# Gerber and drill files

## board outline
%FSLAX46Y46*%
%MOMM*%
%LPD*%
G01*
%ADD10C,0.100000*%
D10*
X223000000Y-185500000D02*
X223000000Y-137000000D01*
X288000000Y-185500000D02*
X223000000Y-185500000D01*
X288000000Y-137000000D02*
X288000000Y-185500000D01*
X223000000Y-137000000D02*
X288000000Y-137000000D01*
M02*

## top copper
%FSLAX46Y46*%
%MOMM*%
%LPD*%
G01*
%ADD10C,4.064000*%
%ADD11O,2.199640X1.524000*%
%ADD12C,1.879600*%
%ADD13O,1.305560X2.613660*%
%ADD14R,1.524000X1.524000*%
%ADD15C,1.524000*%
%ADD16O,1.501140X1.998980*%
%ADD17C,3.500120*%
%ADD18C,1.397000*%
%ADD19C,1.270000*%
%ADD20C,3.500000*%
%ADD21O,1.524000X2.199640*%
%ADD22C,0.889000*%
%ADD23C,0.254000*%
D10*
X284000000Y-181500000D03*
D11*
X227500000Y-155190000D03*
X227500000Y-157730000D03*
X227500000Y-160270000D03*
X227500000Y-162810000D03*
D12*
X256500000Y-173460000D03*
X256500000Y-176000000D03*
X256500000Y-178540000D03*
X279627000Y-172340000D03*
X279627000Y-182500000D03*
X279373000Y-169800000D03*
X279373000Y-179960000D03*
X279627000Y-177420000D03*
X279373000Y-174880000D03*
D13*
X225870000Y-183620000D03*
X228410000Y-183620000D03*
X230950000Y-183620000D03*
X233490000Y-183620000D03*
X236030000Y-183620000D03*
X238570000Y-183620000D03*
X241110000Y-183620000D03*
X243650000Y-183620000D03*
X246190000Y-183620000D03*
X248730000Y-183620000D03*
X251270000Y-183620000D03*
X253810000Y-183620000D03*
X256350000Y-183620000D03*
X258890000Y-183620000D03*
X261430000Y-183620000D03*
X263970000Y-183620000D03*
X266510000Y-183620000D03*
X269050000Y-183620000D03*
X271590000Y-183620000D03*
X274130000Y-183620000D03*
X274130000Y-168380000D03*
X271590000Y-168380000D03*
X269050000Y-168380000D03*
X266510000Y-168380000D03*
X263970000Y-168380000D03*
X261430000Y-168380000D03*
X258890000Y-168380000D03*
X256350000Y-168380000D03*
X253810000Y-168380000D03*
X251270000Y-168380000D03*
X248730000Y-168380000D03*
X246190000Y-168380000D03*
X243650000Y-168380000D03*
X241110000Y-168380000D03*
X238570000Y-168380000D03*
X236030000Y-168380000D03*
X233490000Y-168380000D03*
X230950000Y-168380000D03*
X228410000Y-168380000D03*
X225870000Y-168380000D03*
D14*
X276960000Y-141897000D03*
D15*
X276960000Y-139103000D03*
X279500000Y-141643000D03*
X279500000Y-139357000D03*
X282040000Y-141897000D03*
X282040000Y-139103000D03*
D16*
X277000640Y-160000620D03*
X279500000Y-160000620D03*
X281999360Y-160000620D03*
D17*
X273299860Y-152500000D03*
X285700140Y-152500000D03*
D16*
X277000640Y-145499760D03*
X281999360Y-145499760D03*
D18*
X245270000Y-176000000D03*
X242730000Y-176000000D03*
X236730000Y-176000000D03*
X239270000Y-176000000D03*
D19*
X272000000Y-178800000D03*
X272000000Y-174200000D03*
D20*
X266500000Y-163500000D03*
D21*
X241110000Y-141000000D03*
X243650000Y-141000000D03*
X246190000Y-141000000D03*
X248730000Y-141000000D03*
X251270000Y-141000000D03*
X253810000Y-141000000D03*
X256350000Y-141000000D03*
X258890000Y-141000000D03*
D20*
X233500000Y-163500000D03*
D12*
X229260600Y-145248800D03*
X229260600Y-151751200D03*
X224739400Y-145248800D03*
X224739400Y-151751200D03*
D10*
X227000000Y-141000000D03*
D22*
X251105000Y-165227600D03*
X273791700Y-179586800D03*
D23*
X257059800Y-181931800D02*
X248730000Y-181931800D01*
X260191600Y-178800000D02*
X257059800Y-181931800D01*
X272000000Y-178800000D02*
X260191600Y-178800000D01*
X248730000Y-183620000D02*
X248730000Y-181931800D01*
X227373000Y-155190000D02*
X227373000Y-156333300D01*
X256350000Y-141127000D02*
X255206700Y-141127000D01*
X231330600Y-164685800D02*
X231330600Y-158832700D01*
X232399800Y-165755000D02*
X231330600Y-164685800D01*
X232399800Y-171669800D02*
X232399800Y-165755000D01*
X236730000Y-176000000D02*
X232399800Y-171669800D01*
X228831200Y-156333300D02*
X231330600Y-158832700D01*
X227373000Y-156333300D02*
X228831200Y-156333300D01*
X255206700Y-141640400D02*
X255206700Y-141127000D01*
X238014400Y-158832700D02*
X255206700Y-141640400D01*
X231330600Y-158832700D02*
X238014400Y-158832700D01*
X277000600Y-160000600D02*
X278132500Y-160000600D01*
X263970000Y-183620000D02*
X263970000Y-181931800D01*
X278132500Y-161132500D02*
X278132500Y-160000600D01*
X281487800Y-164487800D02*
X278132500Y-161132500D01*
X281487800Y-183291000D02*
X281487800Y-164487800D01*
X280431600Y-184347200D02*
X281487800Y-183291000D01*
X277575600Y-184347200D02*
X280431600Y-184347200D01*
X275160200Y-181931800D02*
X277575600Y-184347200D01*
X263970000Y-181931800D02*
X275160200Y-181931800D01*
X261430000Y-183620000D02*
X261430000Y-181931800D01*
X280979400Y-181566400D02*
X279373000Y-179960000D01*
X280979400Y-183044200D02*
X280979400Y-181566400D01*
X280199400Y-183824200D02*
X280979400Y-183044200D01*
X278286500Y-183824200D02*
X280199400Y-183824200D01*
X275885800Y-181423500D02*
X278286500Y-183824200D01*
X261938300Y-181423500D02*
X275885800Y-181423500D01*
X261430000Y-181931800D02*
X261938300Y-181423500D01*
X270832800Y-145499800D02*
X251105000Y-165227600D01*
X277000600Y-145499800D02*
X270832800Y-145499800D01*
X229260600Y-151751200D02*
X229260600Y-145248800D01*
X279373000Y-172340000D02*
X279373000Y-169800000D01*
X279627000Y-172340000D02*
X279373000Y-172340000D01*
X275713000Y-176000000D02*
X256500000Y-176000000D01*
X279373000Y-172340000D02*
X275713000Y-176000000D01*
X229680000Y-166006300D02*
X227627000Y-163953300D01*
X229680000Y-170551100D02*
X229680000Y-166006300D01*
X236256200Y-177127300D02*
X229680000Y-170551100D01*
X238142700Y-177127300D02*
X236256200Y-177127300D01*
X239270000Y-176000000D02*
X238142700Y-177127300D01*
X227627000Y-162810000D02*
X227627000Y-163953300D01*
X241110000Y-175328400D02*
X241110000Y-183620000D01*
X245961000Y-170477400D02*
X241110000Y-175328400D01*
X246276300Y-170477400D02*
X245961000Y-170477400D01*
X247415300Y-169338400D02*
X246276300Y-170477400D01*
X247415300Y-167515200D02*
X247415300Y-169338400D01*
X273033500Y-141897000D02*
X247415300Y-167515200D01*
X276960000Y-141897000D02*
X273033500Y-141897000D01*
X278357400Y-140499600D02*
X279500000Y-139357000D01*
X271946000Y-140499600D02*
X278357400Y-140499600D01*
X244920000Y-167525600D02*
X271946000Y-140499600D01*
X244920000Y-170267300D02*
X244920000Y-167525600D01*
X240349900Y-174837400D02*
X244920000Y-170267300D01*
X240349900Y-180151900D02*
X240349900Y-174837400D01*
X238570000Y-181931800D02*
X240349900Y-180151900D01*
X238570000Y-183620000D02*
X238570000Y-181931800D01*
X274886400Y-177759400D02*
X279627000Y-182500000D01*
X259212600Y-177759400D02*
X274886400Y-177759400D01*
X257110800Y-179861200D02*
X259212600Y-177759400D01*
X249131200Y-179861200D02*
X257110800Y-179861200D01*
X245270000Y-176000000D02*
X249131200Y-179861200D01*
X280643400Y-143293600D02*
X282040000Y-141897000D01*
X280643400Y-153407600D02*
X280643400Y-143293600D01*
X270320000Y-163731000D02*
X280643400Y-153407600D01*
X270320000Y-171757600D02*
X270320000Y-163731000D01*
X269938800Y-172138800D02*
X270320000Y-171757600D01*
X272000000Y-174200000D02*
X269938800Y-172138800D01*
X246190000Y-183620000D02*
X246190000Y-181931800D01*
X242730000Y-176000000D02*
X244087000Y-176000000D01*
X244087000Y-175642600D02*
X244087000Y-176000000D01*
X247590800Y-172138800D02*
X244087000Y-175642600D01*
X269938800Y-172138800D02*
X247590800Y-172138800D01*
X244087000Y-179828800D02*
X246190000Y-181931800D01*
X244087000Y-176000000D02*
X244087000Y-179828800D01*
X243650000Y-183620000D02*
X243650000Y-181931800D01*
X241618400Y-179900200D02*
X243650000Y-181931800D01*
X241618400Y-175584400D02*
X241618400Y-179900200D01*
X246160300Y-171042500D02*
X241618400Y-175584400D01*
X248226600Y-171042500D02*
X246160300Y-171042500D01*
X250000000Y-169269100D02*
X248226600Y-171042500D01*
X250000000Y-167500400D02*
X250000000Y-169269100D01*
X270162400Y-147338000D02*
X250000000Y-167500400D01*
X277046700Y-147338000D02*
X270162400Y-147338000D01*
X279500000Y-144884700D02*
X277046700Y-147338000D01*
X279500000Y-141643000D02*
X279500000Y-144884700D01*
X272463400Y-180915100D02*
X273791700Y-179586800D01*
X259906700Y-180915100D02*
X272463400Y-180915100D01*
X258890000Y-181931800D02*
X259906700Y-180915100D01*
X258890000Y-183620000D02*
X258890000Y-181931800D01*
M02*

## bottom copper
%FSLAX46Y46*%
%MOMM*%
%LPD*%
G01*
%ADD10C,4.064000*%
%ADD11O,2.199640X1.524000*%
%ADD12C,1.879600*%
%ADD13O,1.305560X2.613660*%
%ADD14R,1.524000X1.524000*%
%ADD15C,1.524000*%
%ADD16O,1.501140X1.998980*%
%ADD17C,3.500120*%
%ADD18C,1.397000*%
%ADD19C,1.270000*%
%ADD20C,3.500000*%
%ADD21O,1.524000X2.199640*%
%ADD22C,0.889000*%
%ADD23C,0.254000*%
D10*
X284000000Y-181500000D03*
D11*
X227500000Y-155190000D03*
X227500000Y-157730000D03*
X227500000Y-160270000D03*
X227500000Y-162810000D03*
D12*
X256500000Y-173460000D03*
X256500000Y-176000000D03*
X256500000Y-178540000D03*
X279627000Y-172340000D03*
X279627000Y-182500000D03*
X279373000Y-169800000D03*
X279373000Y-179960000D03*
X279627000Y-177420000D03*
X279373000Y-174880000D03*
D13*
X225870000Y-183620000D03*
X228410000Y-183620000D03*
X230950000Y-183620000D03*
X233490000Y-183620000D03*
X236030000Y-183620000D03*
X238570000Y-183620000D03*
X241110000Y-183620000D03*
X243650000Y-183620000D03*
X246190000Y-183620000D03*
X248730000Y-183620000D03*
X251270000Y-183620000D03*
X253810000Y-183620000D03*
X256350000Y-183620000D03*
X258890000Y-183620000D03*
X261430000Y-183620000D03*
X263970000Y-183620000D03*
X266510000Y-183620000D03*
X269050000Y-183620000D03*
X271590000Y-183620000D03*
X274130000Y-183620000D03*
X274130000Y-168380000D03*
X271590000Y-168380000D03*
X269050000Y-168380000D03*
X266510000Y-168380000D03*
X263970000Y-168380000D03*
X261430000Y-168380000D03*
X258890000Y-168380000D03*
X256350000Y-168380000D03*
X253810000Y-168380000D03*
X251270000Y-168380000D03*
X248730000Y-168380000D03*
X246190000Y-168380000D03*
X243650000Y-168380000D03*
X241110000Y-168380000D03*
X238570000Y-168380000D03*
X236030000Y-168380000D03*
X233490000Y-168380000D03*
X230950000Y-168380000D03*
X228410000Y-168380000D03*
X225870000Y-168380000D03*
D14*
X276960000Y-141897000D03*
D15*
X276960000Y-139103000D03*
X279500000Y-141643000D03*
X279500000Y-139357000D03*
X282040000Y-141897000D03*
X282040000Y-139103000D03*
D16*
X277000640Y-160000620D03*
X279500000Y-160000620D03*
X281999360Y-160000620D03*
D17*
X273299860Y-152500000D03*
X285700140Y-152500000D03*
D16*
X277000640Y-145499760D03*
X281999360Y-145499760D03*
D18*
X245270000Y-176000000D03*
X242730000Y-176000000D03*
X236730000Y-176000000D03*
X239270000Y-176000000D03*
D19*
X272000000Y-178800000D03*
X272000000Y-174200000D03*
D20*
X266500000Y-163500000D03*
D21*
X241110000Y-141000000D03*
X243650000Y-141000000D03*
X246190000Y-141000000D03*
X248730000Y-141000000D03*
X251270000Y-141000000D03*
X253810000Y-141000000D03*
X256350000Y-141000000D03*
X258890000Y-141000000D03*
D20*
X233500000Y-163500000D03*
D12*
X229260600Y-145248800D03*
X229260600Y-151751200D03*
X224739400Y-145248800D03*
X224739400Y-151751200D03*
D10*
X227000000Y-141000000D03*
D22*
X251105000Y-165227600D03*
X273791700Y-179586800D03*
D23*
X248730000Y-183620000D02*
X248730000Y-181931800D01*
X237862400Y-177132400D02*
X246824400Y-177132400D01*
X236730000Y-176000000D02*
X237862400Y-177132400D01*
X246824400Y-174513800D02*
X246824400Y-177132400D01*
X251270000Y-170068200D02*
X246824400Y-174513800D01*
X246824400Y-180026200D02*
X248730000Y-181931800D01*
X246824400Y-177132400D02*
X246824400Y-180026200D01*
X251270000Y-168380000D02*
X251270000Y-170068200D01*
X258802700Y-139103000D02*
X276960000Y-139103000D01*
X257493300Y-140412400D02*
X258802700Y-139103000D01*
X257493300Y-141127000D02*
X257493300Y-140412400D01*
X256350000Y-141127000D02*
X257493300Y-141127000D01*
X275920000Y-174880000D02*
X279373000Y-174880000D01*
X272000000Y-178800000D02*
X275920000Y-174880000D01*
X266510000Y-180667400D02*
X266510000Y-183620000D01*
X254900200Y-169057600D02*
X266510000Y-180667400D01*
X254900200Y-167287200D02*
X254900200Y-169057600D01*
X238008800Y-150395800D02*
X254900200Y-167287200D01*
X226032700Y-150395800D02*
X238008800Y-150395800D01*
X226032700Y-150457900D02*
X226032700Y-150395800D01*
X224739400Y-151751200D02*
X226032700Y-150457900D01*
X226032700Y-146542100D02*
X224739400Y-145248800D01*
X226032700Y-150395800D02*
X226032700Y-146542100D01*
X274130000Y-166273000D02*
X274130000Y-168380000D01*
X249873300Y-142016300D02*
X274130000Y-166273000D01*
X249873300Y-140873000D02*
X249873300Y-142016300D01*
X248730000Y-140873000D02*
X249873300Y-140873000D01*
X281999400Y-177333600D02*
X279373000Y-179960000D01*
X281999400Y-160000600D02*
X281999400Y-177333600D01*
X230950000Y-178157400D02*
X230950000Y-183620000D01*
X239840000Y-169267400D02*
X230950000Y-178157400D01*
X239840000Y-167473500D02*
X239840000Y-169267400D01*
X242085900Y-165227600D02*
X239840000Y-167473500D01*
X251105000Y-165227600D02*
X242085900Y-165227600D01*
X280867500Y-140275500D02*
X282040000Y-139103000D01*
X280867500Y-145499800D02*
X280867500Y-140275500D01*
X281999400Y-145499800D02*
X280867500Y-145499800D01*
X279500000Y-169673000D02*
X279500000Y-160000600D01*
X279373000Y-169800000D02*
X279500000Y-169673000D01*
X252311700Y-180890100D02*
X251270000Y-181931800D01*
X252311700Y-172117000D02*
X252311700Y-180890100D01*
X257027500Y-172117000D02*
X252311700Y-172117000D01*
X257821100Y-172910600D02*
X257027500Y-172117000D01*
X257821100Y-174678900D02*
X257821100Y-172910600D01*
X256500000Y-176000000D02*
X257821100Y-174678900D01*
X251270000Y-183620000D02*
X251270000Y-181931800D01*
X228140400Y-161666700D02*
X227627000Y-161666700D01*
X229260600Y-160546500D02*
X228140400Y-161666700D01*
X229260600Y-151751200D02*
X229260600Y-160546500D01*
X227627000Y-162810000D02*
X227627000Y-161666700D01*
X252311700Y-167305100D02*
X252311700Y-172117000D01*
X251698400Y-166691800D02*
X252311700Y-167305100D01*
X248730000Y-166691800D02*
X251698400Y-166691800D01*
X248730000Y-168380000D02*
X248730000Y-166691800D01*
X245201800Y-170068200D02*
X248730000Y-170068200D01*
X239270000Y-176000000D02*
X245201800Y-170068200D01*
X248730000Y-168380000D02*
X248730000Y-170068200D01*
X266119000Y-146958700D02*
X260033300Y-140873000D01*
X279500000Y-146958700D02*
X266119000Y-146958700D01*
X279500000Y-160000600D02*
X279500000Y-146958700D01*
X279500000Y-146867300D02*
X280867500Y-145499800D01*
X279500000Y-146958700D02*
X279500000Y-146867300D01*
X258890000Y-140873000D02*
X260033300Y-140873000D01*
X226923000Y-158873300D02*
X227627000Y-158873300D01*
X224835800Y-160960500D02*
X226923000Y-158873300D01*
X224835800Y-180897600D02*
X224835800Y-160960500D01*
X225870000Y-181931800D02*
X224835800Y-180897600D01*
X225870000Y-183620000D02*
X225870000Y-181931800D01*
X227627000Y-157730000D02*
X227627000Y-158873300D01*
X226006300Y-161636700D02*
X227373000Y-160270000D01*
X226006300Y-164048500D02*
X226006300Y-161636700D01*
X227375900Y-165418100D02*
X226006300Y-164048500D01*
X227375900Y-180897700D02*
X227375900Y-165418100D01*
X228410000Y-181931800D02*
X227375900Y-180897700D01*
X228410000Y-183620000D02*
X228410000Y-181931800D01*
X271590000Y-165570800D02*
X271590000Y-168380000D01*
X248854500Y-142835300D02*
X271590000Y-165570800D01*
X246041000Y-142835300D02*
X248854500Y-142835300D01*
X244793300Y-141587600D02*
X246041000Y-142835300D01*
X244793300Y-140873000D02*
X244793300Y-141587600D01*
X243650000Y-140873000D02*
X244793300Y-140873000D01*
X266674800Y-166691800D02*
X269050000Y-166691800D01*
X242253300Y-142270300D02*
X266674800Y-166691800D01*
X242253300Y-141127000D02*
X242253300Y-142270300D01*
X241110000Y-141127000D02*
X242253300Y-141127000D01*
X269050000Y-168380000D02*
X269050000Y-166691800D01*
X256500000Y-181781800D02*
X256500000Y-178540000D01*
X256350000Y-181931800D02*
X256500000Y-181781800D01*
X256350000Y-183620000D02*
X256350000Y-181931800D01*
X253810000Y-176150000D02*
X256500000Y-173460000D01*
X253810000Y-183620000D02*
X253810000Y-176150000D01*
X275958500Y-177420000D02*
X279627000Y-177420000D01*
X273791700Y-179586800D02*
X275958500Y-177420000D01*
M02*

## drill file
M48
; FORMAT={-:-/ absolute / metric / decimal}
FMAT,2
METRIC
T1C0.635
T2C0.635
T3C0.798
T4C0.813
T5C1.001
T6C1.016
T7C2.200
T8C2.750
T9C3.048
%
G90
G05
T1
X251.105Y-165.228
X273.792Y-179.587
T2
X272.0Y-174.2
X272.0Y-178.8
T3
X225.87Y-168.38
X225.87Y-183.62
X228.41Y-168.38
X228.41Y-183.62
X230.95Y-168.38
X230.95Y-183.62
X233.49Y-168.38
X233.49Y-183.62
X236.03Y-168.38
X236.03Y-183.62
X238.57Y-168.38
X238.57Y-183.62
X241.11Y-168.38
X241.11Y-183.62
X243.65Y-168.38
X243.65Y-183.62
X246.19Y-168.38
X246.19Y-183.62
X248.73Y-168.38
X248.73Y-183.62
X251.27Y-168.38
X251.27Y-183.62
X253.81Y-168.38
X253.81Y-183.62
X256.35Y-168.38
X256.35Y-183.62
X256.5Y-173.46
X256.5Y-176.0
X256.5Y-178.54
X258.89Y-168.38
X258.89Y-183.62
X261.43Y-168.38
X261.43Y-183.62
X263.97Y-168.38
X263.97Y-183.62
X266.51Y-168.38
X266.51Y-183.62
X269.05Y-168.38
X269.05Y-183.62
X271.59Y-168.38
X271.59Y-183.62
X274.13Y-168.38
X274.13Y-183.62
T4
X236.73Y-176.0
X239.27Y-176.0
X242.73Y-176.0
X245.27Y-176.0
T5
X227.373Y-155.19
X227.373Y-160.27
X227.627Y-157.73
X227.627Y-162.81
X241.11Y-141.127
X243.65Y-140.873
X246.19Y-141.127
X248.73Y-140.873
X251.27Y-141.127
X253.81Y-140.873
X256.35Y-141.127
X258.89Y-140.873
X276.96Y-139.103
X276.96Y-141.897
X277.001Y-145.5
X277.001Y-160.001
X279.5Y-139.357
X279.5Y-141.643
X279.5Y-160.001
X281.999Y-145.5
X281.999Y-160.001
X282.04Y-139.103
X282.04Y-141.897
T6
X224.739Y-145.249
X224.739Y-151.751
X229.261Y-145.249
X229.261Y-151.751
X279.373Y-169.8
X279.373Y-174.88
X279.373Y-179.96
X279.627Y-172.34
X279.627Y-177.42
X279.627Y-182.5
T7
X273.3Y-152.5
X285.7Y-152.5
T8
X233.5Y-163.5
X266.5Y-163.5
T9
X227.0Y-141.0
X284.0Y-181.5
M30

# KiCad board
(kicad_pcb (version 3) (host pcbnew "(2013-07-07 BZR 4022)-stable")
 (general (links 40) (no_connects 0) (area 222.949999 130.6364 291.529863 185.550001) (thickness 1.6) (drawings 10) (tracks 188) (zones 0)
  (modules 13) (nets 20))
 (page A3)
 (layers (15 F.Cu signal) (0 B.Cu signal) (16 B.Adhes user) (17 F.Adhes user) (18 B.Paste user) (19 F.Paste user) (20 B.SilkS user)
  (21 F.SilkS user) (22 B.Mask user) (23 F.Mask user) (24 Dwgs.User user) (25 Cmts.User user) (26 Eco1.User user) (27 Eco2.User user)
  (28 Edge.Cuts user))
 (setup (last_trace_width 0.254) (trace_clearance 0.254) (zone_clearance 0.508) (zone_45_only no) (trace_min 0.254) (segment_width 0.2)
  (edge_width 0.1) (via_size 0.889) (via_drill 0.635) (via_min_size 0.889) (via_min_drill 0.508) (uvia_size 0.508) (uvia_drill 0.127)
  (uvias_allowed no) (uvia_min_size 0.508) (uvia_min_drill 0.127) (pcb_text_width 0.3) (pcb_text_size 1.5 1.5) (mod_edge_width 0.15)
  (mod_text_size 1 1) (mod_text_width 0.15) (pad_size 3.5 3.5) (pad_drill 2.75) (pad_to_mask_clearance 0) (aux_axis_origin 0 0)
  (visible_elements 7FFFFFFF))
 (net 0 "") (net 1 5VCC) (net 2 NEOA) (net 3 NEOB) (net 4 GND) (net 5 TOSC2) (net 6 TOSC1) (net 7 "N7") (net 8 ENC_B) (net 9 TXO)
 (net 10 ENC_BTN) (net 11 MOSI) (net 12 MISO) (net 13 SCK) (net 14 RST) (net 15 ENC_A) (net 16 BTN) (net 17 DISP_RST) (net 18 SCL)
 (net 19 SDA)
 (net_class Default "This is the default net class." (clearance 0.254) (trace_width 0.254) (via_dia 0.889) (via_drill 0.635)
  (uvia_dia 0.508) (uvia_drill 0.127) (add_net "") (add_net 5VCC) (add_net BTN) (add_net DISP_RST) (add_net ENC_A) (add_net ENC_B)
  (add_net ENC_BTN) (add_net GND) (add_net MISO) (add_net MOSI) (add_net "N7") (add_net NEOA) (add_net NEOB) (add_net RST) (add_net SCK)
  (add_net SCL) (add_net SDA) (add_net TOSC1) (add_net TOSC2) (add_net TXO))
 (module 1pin (layer F.Cu) (at 284 181.5)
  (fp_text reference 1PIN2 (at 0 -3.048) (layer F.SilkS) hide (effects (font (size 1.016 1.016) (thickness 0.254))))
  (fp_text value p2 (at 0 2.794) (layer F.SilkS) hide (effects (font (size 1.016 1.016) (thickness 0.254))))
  (pad 1 thru_hole circle (at 0 0) (size 4.064 4.064) (drill 3.048) (layers *.Cu *.Mask F.SilkS)))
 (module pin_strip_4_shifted (layer F.Cu) (at 227.5 159 270)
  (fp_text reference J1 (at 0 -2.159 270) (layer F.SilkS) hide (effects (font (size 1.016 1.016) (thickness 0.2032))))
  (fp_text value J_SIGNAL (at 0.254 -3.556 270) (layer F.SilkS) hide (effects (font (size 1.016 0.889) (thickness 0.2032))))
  (pad 1 thru_hole oval (at -3.81 0.127 270) (size 1.524 2.19964) (drill 1.00076 (offset 0 -0.127)) (layers *.Cu *.Mask F.SilkS)
   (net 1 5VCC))
  (pad 2 thru_hole oval (at -1.27 -0.127 270) (size 1.524 2.19964) (drill 1.00076 (offset 0 0.127)) (layers *.Cu *.Mask F.SilkS)
   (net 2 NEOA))
  (pad 3 thru_hole oval (at 1.27 0.127 270) (size 1.524 2.19964) (drill 1.00076 (offset 0 -0.127)) (layers *.Cu *.Mask F.SilkS) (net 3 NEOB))
  (pad 4 thru_hole oval (at 3.81 -0.127 270) (size 1.524 2.19964) (drill 1.00076 (offset 0 0.127)) (layers *.Cu *.Mask F.SilkS) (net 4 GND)))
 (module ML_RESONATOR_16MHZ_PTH (layer F.Cu) (at 256.5 176 270)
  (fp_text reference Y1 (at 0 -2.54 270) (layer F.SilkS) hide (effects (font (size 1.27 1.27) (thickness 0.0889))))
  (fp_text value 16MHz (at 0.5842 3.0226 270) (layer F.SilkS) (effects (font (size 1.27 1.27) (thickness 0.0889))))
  (pad 1 thru_hole circle (at -2.54 0 270) (size 1.8796 1.8796) (drill 0.79756) (layers *.Cu *.Mask F.Paste F.SilkS) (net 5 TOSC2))
  (pad 2 thru_hole circle (at 0 0 270) (size 1.8796 1.8796) (drill 0.79756) (layers *.Cu *.Mask F.Paste F.SilkS) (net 4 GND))
  (pad 3 thru_hole circle (at 2.54 0 270) (size 1.8796 1.8796) (drill 0.79756) (layers *.Cu *.Mask F.Paste F.SilkS) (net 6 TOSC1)))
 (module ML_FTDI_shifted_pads (layer F.Cu) (at 279.5 182.5 90)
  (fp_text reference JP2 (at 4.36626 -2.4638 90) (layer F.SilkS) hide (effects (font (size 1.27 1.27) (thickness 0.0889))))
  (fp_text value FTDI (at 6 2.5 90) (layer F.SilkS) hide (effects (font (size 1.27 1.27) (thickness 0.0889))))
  (pad CTS thru_hole circle (at 10.16 0.127 90) (size 1.8796 1.8796) (drill 1.016) (layers *.Cu *.Mask F.Paste F.SilkS) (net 4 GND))
  (pad DTR thru_hole circle (at 0 0.127 90) (size 1.8796 1.8796) (drill 1.016) (layers *.Cu *.Mask F.Paste F.SilkS) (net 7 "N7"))
  (pad GND thru_hole circle (at 12.7 -0.127 90) (size 1.8796 1.8796) (drill 1.016) (layers *.Cu *.Mask F.Paste F.SilkS) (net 4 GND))
  (pad RXI thru_hole circle (at 2.54 -0.127 90) (size 1.8796 1.8796) (drill 1.016) (layers *.Cu *.Mask F.Paste F.SilkS) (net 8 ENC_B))
  (pad TXO thru_hole circle (at 5.08 0.127 90) (size 1.8796 1.8796) (drill 1.016) (layers *.Cu *.Mask F.Paste F.SilkS) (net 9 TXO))
  (pad VCC thru_hole circle (at 7.62 -0.127 90) (size 1.8796 1.8796) (drill 1.016) (layers *.Cu *.Mask F.Paste F.SilkS) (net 1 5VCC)))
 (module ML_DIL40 (layer F.Cu) (at 250 176)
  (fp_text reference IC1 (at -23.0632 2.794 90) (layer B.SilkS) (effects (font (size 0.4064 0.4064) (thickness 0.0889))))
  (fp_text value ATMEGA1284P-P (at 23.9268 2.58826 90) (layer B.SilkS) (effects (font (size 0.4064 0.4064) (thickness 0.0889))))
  (pad 1 thru_hole oval (at -24.13 7.62) (size 1.30556 2.61366) (drill 0.79756) (layers *.Cu *.Mask F.Paste F.SilkS) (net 2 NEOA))
  (pad 2 thru_hole oval (at -21.59 7.62) (size 1.30556 2.61366) (drill 0.79756) (layers *.Cu *.Mask F.Paste F.SilkS) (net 3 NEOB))
  (pad 3 thru_hole oval (at -19.05 7.62) (size 1.30556 2.61366) (drill 0.79756) (layers *.Cu *.Mask F.Paste F.SilkS) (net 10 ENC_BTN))
  (pad 4 thru_hole oval (at -16.51 7.62) (size 1.30556 2.61366) (drill 0.79756) (layers *.Cu *.Mask F.Paste F.SilkS))
  (pad 5 thru_hole oval (at -13.97 7.62) (size 1.30556 2.61366) (drill 0.79756) (layers *.Cu *.Mask F.Paste F.SilkS))
  (pad 6 thru_hole oval (at -11.43 7.62) (size 1.30556 2.61366) (drill 0.79756) (layers *.Cu *.Mask F.Paste F.SilkS) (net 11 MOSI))
  (pad 7 thru_hole oval (at -8.89 7.62) (size 1.30556 2.61366) (drill 0.79756) (layers *.Cu *.Mask F.Paste F.SilkS) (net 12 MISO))
  (pad 8 thru_hole oval (at -6.35 7.62) (size 1.30556 2.61366) (drill 0.79756) (layers *.Cu *.Mask F.Paste F.SilkS) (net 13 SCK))
  (pad 9 thru_hole oval (at -3.81 7.62) (size 1.30556 2.61366) (drill 0.79756) (layers *.Cu *.Mask F.Paste F.SilkS) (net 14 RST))
  (pad 10 thru_hole oval (at -1.27 7.62) (size 1.30556 2.61366) (drill 0.79756) (layers *.Cu *.Mask F.Paste F.SilkS) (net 1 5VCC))
  (pad 11 thru_hole oval (at 1.27 7.62) (size 1.30556 2.61366) (drill 0.79756) (layers *.Cu *.Mask F.Paste F.SilkS) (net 4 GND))
  (pad 12 thru_hole oval (at 3.81 7.62) (size 1.30556 2.61366) (drill 0.79756) (layers *.Cu *.Mask F.Paste F.SilkS) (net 5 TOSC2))
  (pad 13 thru_hole oval (at 6.35 7.62) (size 1.30556 2.61366) (drill 0.79756) (layers *.Cu *.Mask F.Paste F.SilkS) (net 6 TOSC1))
  (pad 14 thru_hole oval (at 8.89 7.62) (size 1.30556 2.61366) (drill 0.79756) (layers *.Cu *.Mask F.Paste F.SilkS) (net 9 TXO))
  (pad 15 thru_hole oval (at 11.43 7.62) (size 1.30556 2.61366) (drill 0.79756) (layers *.Cu *.Mask F.Paste F.SilkS) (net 8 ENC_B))
  (pad 16 thru_hole oval (at 13.97 7.62) (size 1.30556 2.61366) (drill 0.79756) (layers *.Cu *.Mask F.Paste F.SilkS) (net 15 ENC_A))
  (pad 17 thru_hole oval (at 16.51 7.62) (size 1.30556 2.61366) (drill 0.79756) (layers *.Cu *.Mask F.Paste F.SilkS) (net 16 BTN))
  (pad 18 thru_hole oval (at 19.05 7.62) (size 1.30556 2.61366) (drill 0.79756) (layers *.Cu *.Mask F.Paste F.SilkS))
  (pad 19 thru_hole oval (at 21.59 7.62) (size 1.30556 2.61366) (drill 0.79756) (layers *.Cu *.Mask F.Paste F.SilkS))
  (pad 20 thru_hole oval (at 24.13 7.62) (size 1.30556 2.61366) (drill 0.79756) (layers *.Cu *.Mask F.Paste F.SilkS))
  (pad 21 thru_hole oval (at 24.13 -7.62) (size 1.30556 2.61366) (drill 0.79756) (layers *.Cu *.Mask F.Paste F.SilkS) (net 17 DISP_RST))
  (pad 22 thru_hole oval (at 21.59 -7.62) (size 1.30556 2.61366) (drill 0.79756) (layers *.Cu *.Mask F.Paste F.SilkS) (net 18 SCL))
  (pad 23 thru_hole oval (at 19.05 -7.62) (size 1.30556 2.61366) (drill 0.79756) (layers *.Cu *.Mask F.Paste F.SilkS) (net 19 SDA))
  (pad 24 thru_hole oval (at 16.51 -7.62) (size 1.30556 2.61366) (drill 0.79756) (layers *.Cu *.Mask F.Paste F.SilkS))
  (pad 25 thru_hole oval (at 13.97 -7.62) (size 1.30556 2.61366) (drill 0.79756) (layers *.Cu *.Mask F.Paste F.SilkS))
  (pad 26 thru_hole oval (at 11.43 -7.62) (size 1.30556 2.61366) (drill 0.79756) (layers *.Cu *.Mask F.Paste F.SilkS))
  (pad 27 thru_hole oval (at 8.89 -7.62) (size 1.30556 2.61366) (drill 0.79756) (layers *.Cu *.Mask F.Paste F.SilkS))
  (pad 28 thru_hole oval (at 6.35 -7.62) (size 1.30556 2.61366) (drill 0.79756) (layers *.Cu *.Mask F.Paste F.SilkS))
  (pad 29 thru_hole oval (at 3.81 -7.62) (size 1.30556 2.61366) (drill 0.79756) (layers *.Cu *.Mask F.Paste F.SilkS))
  (pad 30 thru_hole oval (at 1.27 -7.62) (size 1.30556 2.61366) (drill 0.79756) (layers *.Cu *.Mask F.Paste F.SilkS) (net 1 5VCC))
  (pad 31 thru_hole oval (at -1.27 -7.62) (size 1.30556 2.61366) (drill 0.79756) (layers *.Cu *.Mask F.Paste F.SilkS) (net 4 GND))
  (pad 32 thru_hole oval (at -3.81 -7.62) (size 1.30556 2.61366) (drill 0.79756) (layers *.Cu *.Mask F.Paste F.SilkS))
  (pad 33 thru_hole oval (at -6.35 -7.62) (size 1.30556 2.61366) (drill 0.79756) (layers *.Cu *.Mask F.Paste F.SilkS))
  (pad 34 thru_hole oval (at -8.89 -7.62) (size 1.30556 2.61366) (drill 0.79756) (layers *.Cu *.Mask F.Paste F.SilkS))
  (pad 35 thru_hole oval (at -11.43 -7.62) (size 1.30556 2.61366) (drill 0.79756) (layers *.Cu *.Mask F.Paste F.SilkS))
  (pad 36 thru_hole oval (at -13.97 -7.62) (size 1.30556 2.61366) (drill 0.79756) (layers *.Cu *.Mask F.Paste F.SilkS))
  (pad 37 thru_hole oval (at -16.51 -7.62) (size 1.30556 2.61366) (drill 0.79756) (layers *.Cu *.Mask F.Paste F.SilkS))
  (pad 38 thru_hole oval (at -19.05 -7.62) (size 1.30556 2.61366) (drill 0.79756) (layers *.Cu *.Mask F.Paste F.SilkS))
  (pad 39 thru_hole oval (at -21.59 -7.62) (size 1.30556 2.61366) (drill 0.79756) (layers *.Cu *.Mask F.Paste F.SilkS))
  (pad 40 thru_hole oval (at -24.13 -7.62) (size 1.30556 2.61366) (drill 0.79756) (layers *.Cu *.Mask F.Paste F.SilkS)))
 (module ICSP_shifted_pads (layer F.Cu) (at 279.5 140.5)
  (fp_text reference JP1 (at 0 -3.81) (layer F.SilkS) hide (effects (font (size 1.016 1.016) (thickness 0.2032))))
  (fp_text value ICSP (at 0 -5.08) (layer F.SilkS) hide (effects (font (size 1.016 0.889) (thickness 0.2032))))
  (pad 1 thru_hole rect (at -2.54 1.397) (size 1.524 1.524) (drill 1.00076) (layers *.Cu *.Mask F.SilkS) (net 12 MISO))
  (pad 2 thru_hole circle (at -2.54 -1.397) (size 1.524 1.524) (drill 1.00076) (layers *.Cu *.Mask F.SilkS) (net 1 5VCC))
  (pad 3 thru_hole circle (at 0 1.143) (size 1.524 1.524) (drill 1.00076) (layers *.Cu *.Mask F.SilkS) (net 13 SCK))
  (pad 4 thru_hole circle (at 0 -1.143) (size 1.524 1.524) (drill 1.00076) (layers *.Cu *.Mask F.SilkS) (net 11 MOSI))
  (pad 5 thru_hole circle (at 2.54 1.397) (size 1.524 1.524) (drill 1.00076) (layers *.Cu *.Mask F.SilkS) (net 14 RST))
  (pad 6 thru_hole circle (at 2.54 -1.397) (size 1.524 1.524) (drill 1.00076) (layers *.Cu *.Mask F.SilkS) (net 4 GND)))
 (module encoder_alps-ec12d (layer F.Cu) (at 279.5 152.5) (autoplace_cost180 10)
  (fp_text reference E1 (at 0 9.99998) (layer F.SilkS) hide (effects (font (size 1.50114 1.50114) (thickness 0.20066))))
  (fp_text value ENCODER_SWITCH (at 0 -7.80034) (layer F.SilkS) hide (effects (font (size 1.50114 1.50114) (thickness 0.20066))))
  (pad 1 thru_hole oval (at -2.49936 7.50062) (size 1.50114 1.99898) (drill 1.00076) (layers *.Cu *.Mask F.SilkS) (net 15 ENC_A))
  (pad 2 thru_hole oval (at 0 7.50062) (size 1.50114 1.99898) (drill 1.00076) (layers *.Cu *.Mask F.SilkS) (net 4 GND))
  (pad 3 thru_hole oval (at 2.49936 7.50062) (size 1.50114 1.99898) (drill 1.00076) (layers *.Cu *.Mask F.SilkS) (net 8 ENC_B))
  (pad "" thru_hole circle (at -6.20014 0) (size 3.50012 3.50012) (drill 2.19964) (layers *.Cu *.Mask F.SilkS))
  (pad "" thru_hole circle (at 6.20014 0) (size 3.50012 3.50012) (drill 2.19964) (layers *.Cu *.Mask F.SilkS))
  (pad 5 thru_hole oval (at -2.49936 -7.00024) (size 1.50114 1.99898) (drill 1.00076) (layers *.Cu *.Mask F.SilkS) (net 10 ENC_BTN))
  (pad 4 thru_hole oval (at 2.49936 -7.00024) (size 1.50114 1.99898) (drill 1.00076) (layers *.Cu *.Mask F.SilkS) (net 4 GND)))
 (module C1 (layer F.Cu) (at 244 176 180)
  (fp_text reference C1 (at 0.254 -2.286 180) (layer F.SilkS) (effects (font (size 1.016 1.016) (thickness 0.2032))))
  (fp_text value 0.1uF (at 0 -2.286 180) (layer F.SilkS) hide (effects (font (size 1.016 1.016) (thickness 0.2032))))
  (pad 1 thru_hole circle (at -1.27 0 180) (size 1.397 1.397) (drill 0.8128) (layers *.Cu *.Mask F.SilkS) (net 7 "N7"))
  (pad 2 thru_hole circle (at 1.27 0 180) (size 1.397 1.397) (drill 0.8128) (layers *.Cu *.Mask F.SilkS) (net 14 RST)))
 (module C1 (layer F.Cu) (at 238 176)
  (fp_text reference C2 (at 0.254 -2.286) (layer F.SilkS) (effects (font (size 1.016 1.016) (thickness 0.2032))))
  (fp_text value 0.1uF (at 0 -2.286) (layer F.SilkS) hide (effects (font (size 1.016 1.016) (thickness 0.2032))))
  (pad 1 thru_hole circle (at -1.27 0) (size 1.397 1.397) (drill 0.8128) (layers *.Cu *.Mask F.SilkS) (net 1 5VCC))
  (pad 2 thru_hole circle (at 1.27 0) (size 1.397 1.397) (drill 0.8128) (layers *.Cu *.Mask F.SilkS) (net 4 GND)))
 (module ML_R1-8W (layer F.Cu) (at 272 176.5 90)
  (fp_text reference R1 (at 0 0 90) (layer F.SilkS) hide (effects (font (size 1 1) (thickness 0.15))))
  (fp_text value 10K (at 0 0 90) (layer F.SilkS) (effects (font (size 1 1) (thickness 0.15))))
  (pad 1 thru_hole circle (at -2.3 0 90) (size 1.27 1.27) (drill 0.635) (layers *.Cu *.Mask F.SilkS) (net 1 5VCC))
  (pad 2 thru_hole circle (at 2.3 0 90) (size 1.27 1.27) (drill 0.635) (layers *.Cu *.Mask F.SilkS) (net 14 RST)))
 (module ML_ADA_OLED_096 (layer F.Cu) (at 250 141)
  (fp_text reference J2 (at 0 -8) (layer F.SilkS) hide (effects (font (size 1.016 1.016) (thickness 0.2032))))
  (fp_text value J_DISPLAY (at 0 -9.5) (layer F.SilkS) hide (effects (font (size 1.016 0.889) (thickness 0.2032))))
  (pad 9 thru_hole circle (at 16.5 22.5) (size 3.5 3.5) (drill 2.75) (layers *.Cu *.Mask F.SilkS))
  (pad 1 thru_hole oval (at -8.89 0.127) (size 1.524 2.19964) (drill 1.00076 (offset 0 -0.127)) (layers *.Cu *.Mask F.SilkS) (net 19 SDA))
  (pad 2 thru_hole oval (at -6.35 -0.127) (size 1.524 2.19964) (drill 1.00076 (offset 0 0.127)) (layers *.Cu *.Mask F.SilkS) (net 18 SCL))
  (pad 3 thru_hole oval (at -3.81 0.127) (size 1.524 2.19964) (drill 1.00076 (offset 0 -0.127)) (layers *.Cu *.Mask F.SilkS))
  (pad 4 thru_hole oval (at -1.27 -0.127) (size 1.524 2.19964) (drill 1.00076 (offset 0 0.127)) (layers *.Cu *.Mask F.SilkS)
   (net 17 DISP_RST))
  (pad 5 thru_hole oval (at 1.27 0.127) (size 1.524 2.19964) (drill 1.00076 (offset 0 -0.127)) (layers *.Cu *.Mask F.SilkS))
  (pad 6 thru_hole oval (at 3.81 -0.127) (size 1.524 2.19964) (drill 1.00076 (offset 0 0.127)) (layers *.Cu *.Mask F.SilkS))
  (pad 7 thru_hole oval (at 6.35 0.127) (size 1.524 2.19964) (drill 1.00076 (offset 0 -0.127)) (layers *.Cu *.Mask F.SilkS) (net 1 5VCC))
  (pad 8 thru_hole oval (at 8.89 -0.127) (size 1.524 2.19964) (drill 1.00076 (offset 0 0.127)) (layers *.Cu *.Mask F.SilkS) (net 4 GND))
  (pad 9 thru_hole circle (at -16.5 22.5) (size 3.5 3.5) (drill 2.75) (layers *.Cu *.Mask F.SilkS)))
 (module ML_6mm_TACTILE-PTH (layer F.Cu) (at 227 148.5 270)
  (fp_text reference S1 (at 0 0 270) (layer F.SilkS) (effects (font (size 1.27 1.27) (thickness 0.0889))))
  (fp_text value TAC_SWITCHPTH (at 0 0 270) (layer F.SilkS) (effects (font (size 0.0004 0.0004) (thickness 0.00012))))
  (pad 1 thru_hole circle (at -3.2512 -2.2606 270) (size 1.8796 1.8796) (drill 1.016) (layers *.Cu *.Mask F.Paste F.SilkS) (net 4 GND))
  (pad 2 thru_hole circle (at 3.2512 -2.2606 270) (size 1.8796 1.8796) (drill 1.016) (layers *.Cu *.Mask F.Paste F.SilkS) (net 4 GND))
  (pad 3 thru_hole circle (at -3.2512 2.2606 270) (size 1.8796 1.8796) (drill 1.016) (layers *.Cu *.Mask F.Paste F.SilkS) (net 16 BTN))
  (pad 4 thru_hole circle (at 3.2512 2.2606 270) (size 1.8796 1.8796) (drill 1.016) (layers *.Cu *.Mask F.Paste F.SilkS) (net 16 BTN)))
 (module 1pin (layer F.Cu) (at 227 141)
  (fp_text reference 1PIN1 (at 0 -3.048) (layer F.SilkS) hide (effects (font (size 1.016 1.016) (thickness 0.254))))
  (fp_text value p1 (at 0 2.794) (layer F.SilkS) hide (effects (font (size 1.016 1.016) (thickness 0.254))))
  (pad 1 thru_hole circle (at 0 0) (size 4.064 4.064) (drill 3.048) (layers *.Cu *.Mask F.SilkS)))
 (gr_line (start 223 185.5) (end 223 137) (angle 90) (layer Edge.Cuts) (width 0.1))
 (gr_line (start 288 185.5) (end 223 185.5) (angle 90) (layer Edge.Cuts) (width 0.1))
 (gr_line (start 288 137) (end 288 185.5) (angle 90) (layer Edge.Cuts) (width 0.1))
 (gr_line (start 223 137) (end 288 137) (angle 90) (layer Edge.Cuts) (width 0.1))
 (segment (start 248.73 183.62) (end 248.73 181.9318) (width 0.254) (layer B.Cu) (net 1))
 (segment (start 237.8624 177.1324) (end 246.8244 177.1324) (width 0.254) (layer B.Cu) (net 1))
 (segment (start 236.73 176) (end 237.8624 177.1324) (width 0.254) (layer B.Cu) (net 1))
 (segment (start 246.8244 174.5138) (end 246.8244 177.1324) (width 0.254) (layer B.Cu) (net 1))
 (segment (start 251.27 170.0682) (end 246.8244 174.5138) (width 0.254) (layer B.Cu) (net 1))
 (segment (start 246.8244 180.0262) (end 248.73 181.9318) (width 0.254) (layer B.Cu) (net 1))
 (segment (start 246.8244 177.1324) (end 246.8244 180.0262) (width 0.254) (layer B.Cu) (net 1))
 (segment (start 251.27 168.38) (end 251.27 170.0682) (width 0.254) (layer B.Cu) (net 1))
 (segment (start 257.0598 181.9318) (end 248.73 181.9318) (width 0.254) (layer F.Cu) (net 1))
 (segment (start 260.1916 178.8) (end 257.0598 181.9318) (width 0.254) (layer F.Cu) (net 1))
 (segment (start 272 178.8) (end 260.1916 178.8) (width 0.254) (layer F.Cu) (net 1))
 (segment (start 248.73 183.62) (end 248.73 181.9318) (width 0.254) (layer F.Cu) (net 1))
 (segment (start 227.373 155.19) (end 227.373 156.3333) (width 0.254) (layer F.Cu) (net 1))
 (segment (start 258.8027 139.103) (end 276.96 139.103) (width 0.254) (layer B.Cu) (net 1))
 (segment (start 257.4933 140.4124) (end 258.8027 139.103) (width 0.254) (layer B.Cu) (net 1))
 (segment (start 257.4933 141.127) (end 257.4933 140.4124) (width 0.254) (layer B.Cu) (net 1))
 (segment (start 256.35 141.127) (end 257.4933 141.127) (width 0.254) (layer B.Cu) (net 1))
 (segment (start 256.35 141.127) (end 255.2067 141.127) (width 0.254) (layer F.Cu) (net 1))
 (segment (start 231.3306 164.6858) (end 231.3306 158.8327) (width 0.254) (layer F.Cu) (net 1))
 (segment (start 232.3998 165.755) (end 231.3306 164.6858) (width 0.254) (layer F.Cu) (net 1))
 (segment (start 232.3998 171.6698) (end 232.3998 165.755) (width 0.254) (layer F.Cu) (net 1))
 (segment (start 236.73 176) (end 232.3998 171.6698) (width 0.254) (layer F.Cu) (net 1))
 (segment (start 228.8312 156.3333) (end 231.3306 158.8327) (width 0.254) (layer F.Cu) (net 1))
 (segment (start 227.373 156.3333) (end 228.8312 156.3333) (width 0.254) (layer F.Cu) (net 1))
 (segment (start 255.2067 141.6404) (end 255.2067 141.127) (width 0.254) (layer F.Cu) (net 1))
 (segment (start 238.0144 158.8327) (end 255.2067 141.6404) (width 0.254) (layer F.Cu) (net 1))
 (segment (start 231.3306 158.8327) (end 238.0144 158.8327) (width 0.254) (layer F.Cu) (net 1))
 (segment (start 275.92 174.88) (end 279.373 174.88) (width 0.254) (layer B.Cu) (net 1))
 (segment (start 272 178.8) (end 275.92 174.88) (width 0.254) (layer B.Cu) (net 1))
 (segment (start 266.51 180.6674) (end 266.51 183.62) (width 0.254) (layer B.Cu) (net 16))
 (segment (start 254.9002 169.0576) (end 266.51 180.6674) (width 0.254) (layer B.Cu) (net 16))
 (segment (start 254.9002 167.2872) (end 254.9002 169.0576) (width 0.254) (layer B.Cu) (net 16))
 (segment (start 238.0088 150.3958) (end 254.9002 167.2872) (width 0.254) (layer B.Cu) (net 16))
 (segment (start 226.0327 150.3958) (end 238.0088 150.3958) (width 0.254) (layer B.Cu) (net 16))
 (segment (start 226.0327 150.4579) (end 226.0327 150.3958) (width 0.254) (layer B.Cu) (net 16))
 (segment (start 224.7394 151.7512) (end 226.0327 150.4579) (width 0.254) (layer B.Cu) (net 16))
 (segment (start 226.0327 146.5421) (end 224.7394 145.2488) (width 0.254) (layer B.Cu) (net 16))
 (segment (start 226.0327 150.3958) (end 226.0327 146.5421) (width 0.254) (layer B.Cu) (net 16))
 (segment (start 274.13 166.273) (end 274.13 168.38) (width 0.254) (layer B.Cu) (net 17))
 (segment (start 249.8733 142.0163) (end 274.13 166.273) (width 0.254) (layer B.Cu) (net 17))
 (segment (start 249.8733 140.873) (end 249.8733 142.0163) (width 0.254) (layer B.Cu) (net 17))
 (segment (start 248.73 140.873) (end 249.8733 140.873) (width 0.254) (layer B.Cu) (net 17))
 (segment (start 277.0006 160.0006) (end 278.1325 160.0006) (width 0.254) (layer F.Cu) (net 15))
 (segment (start 263.97 183.62) (end 263.97 181.9318) (width 0.254) (layer F.Cu) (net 15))
 (segment (start 278.1325 161.1325) (end 278.1325 160.0006) (width 0.254) (layer F.Cu) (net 15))
 (segment (start 281.4878 164.4878) (end 278.1325 161.1325) (width 0.254) (layer F.Cu) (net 15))
 (segment (start 281.4878 183.291) (end 281.4878 164.4878) (width 0.254) (layer F.Cu) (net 15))
 (segment (start 280.4316 184.3472) (end 281.4878 183.291) (width 0.254) (layer F.Cu) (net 15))
 (segment (start 277.5756 184.3472) (end 280.4316 184.3472) (width 0.254) (layer F.Cu) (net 15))
 (segment (start 275.1602 181.9318) (end 277.5756 184.3472) (width 0.254) (layer F.Cu) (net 15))
 (segment (start 263.97 181.9318) (end 275.1602 181.9318) (width 0.254) (layer F.Cu) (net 15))
 (segment (start 261.43 183.62) (end 261.43 181.9318) (width 0.254) (layer F.Cu) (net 8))
 (segment (start 281.9994 177.3336) (end 279.373 179.96) (width 0.254) (layer B.Cu) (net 8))
 (segment (start 281.9994 160.0006) (end 281.9994 177.3336) (width 0.254) (layer B.Cu) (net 8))
 (segment (start 280.9794 181.5664) (end 279.373 179.96) (width 0.254) (layer F.Cu) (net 8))
 (segment (start 280.9794 183.0442) (end 280.9794 181.5664) (width 0.254) (layer F.Cu) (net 8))
 (segment (start 280.1994 183.8242) (end 280.9794 183.0442) (width 0.254) (layer F.Cu) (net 8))
 (segment (start 278.2865 183.8242) (end 280.1994 183.8242) (width 0.254) (layer F.Cu) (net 8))
 (segment (start 275.8858 181.4235) (end 278.2865 183.8242) (width 0.254) (layer F.Cu) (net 8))
 (segment (start 261.9383 181.4235) (end 275.8858 181.4235) (width 0.254) (layer F.Cu) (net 8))
 (segment (start 261.43 181.9318) (end 261.9383 181.4235) (width 0.254) (layer F.Cu) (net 8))
 (via (at 251.105 165.2276) (size 0.889) (layers F.Cu B.Cu) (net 10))
 (segment (start 270.8328 145.4998) (end 251.105 165.2276) (width 0.254) (layer F.Cu) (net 10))
 (segment (start 277.0006 145.4998) (end 270.8328 145.4998) (width 0.254) (layer F.Cu) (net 10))
 (segment (start 230.95 178.1574) (end 230.95 183.62) (width 0.254) (layer B.Cu) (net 10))
 (segment (start 239.84 169.2674) (end 230.95 178.1574) (width 0.254) (layer B.Cu) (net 10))
 (segment (start 239.84 167.4735) (end 239.84 169.2674) (width 0.254) (layer B.Cu) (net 10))
 (segment (start 242.0859 165.2276) (end 239.84 167.4735) (width 0.254) (layer B.Cu) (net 10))
 (segment (start 251.105 165.2276) (end 242.0859 165.2276) (width 0.254) (layer B.Cu) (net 10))
 (segment (start 229.2606 151.7512) (end 229.2606 145.2488) (width 0.254) (layer F.Cu) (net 4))
 (segment (start 279.373 172.34) (end 279.373 169.8) (width 0.254) (layer F.Cu) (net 4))
 (segment (start 279.627 172.34) (end 279.373 172.34) (width 0.254) (layer F.Cu) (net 4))
 (segment (start 275.713 176) (end 256.5 176) (width 0.254) (layer F.Cu) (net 4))
 (segment (start 279.373 172.34) (end 275.713 176) (width 0.254) (layer F.Cu) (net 4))
 (segment (start 280.8675 140.2755) (end 282.04 139.103) (width 0.254) (layer B.Cu) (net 4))
 (segment (start 280.8675 145.4998) (end 280.8675 140.2755) (width 0.254) (layer B.Cu) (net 4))
 (segment (start 281.9994 145.4998) (end 280.8675 145.4998) (width 0.254) (layer B.Cu) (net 4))
 (segment (start 279.5 169.673) (end 279.5 160.0006) (width 0.254) (layer B.Cu) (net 4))
 (segment (start 279.373 169.8) (end 279.5 169.673) (width 0.254) (layer B.Cu) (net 4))
 (segment (start 252.3117 180.8901) (end 251.27 181.9318) (width 0.254) (layer B.Cu) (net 4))
 (segment (start 252.3117 172.117) (end 252.3117 180.8901) (width 0.254) (layer B.Cu) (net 4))
 (segment (start 257.0275 172.117) (end 252.3117 172.117) (width 0.254) (layer B.Cu) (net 4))
 (segment (start 257.8211 172.9106) (end 257.0275 172.117) (width 0.254) (layer B.Cu) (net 4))
 (segment (start 257.8211 174.6789) (end 257.8211 172.9106) (width 0.254) (layer B.Cu) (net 4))
 (segment (start 256.5 176) (end 257.8211 174.6789) (width 0.254) (layer B.Cu) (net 4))
 (segment (start 251.27 183.62) (end 251.27 181.9318) (width 0.254) (layer B.Cu) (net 4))
 (segment (start 228.1404 161.6667) (end 227.627 161.6667) (width 0.254) (layer B.Cu) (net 4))
 (segment (start 229.2606 160.5465) (end 228.1404 161.6667) (width 0.254) (layer B.Cu) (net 4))
 (segment (start 229.2606 151.7512) (end 229.2606 160.5465) (width 0.254) (layer B.Cu) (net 4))
 (segment (start 227.627 162.81) (end 227.627 161.6667) (width 0.254) (layer B.Cu) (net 4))
 (segment (start 229.68 166.0063) (end 227.627 163.9533) (width 0.254) (layer F.Cu) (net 4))
 (segment (start 229.68 170.5511) (end 229.68 166.0063) (width 0.254) (layer F.Cu) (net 4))
 (segment (start 236.2562 177.1273) (end 229.68 170.5511) (width 0.254) (layer F.Cu) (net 4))
 (segment (start 238.1427 177.1273) (end 236.2562 177.1273) (width 0.254) (layer F.Cu) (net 4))
 (segment (start 239.27 176) (end 238.1427 177.1273) (width 0.254) (layer F.Cu) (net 4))
 (segment (start 227.627 162.81) (end 227.627 163.9533) (width 0.254) (layer F.Cu) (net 4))
 (segment (start 252.3117 167.3051) (end 252.3117 172.117) (width 0.254) (layer B.Cu) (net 4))
 (segment (start 251.6984 166.6918) (end 252.3117 167.3051) (width 0.254) (layer B.Cu) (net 4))
 (segment (start 248.73 166.6918) (end 251.6984 166.6918) (width 0.254) (layer B.Cu) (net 4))
 (segment (start 248.73 168.38) (end 248.73 166.6918) (width 0.254) (layer B.Cu) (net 4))
 (segment (start 245.2018 170.0682) (end 248.73 170.0682) (width 0.254) (layer B.Cu) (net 4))
 (segment (start 239.27 176) (end 245.2018 170.0682) (width 0.254) (layer B.Cu) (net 4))
 (segment (start 248.73 168.38) (end 248.73 170.0682) (width 0.254) (layer B.Cu) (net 4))
 (segment (start 266.119 146.9587) (end 260.0333 140.873) (width 0.254) (layer B.Cu) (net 4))
 (segment (start 279.5 146.9587) (end 266.119 146.9587) (width 0.254) (layer B.Cu) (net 4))
 (segment (start 279.5 160.0006) (end 279.5 146.9587) (width 0.254) (layer B.Cu) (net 4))
 (segment (start 279.5 146.8673) (end 280.8675 145.4998) (width 0.254) (layer B.Cu) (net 4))
 (segment (start 279.5 146.9587) (end 279.5 146.8673) (width 0.254) (layer B.Cu) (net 4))
 (segment (start 258.89 140.873) (end 260.0333 140.873) (width 0.254) (layer B.Cu) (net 4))
 (segment (start 241.11 175.3284) (end 241.11 183.62) (width 0.254) (layer F.Cu) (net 12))
 (segment (start 245.961 170.4774) (end 241.11 175.3284) (width 0.254) (layer F.Cu) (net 12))
 (segment (start 246.2763 170.4774) (end 245.961 170.4774) (width 0.254) (layer F.Cu) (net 12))
 (segment (start 247.4153 169.3384) (end 246.2763 170.4774) (width 0.254) (layer F.Cu) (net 12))
 (segment (start 247.4153 167.5152) (end 247.4153 169.3384) (width 0.254) (layer F.Cu) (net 12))
 (segment (start 273.0335 141.897) (end 247.4153 167.5152) (width 0.254) (layer F.Cu) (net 12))
 (segment (start 276.96 141.897) (end 273.0335 141.897) (width 0.254) (layer F.Cu) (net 12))
 (segment (start 278.3574 140.4996) (end 279.5 139.357) (width 0.254) (layer F.Cu) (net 11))
 (segment (start 271.946 140.4996) (end 278.3574 140.4996) (width 0.254) (layer F.Cu) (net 11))
 (segment (start 244.92 167.5256) (end 271.946 140.4996) (width 0.254) (layer F.Cu) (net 11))
 (segment (start 244.92 170.2673) (end 244.92 167.5256) (width 0.254) (layer F.Cu) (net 11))
 (segment (start 240.3499 174.8374) (end 244.92 170.2673) (width 0.254) (layer F.Cu) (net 11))
 (segment (start 240.3499 180.1519) (end 240.3499 174.8374) (width 0.254) (layer F.Cu) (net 11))
 (segment (start 238.57 181.9318) (end 240.3499 180.1519) (width 0.254) (layer F.Cu) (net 11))
 (segment (start 238.57 183.62) (end 238.57 181.9318) (width 0.254) (layer F.Cu) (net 11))
 (segment (start 274.8864 177.7594) (end 279.627 182.5) (width 0.254) (layer F.Cu) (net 7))
 (segment (start 259.2126 177.7594) (end 274.8864 177.7594) (width 0.254) (layer F.Cu) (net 7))
 (segment (start 257.1108 179.8612) (end 259.2126 177.7594) (width 0.254) (layer F.Cu) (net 7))
 (segment (start 249.1312 179.8612) (end 257.1108 179.8612) (width 0.254) (layer F.Cu) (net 7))
 (segment (start 245.27 176) (end 249.1312 179.8612) (width 0.254) (layer F.Cu) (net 7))
 (segment (start 226.923 158.8733) (end 227.627 158.8733) (width 0.254) (layer B.Cu) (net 2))
 (segment (start 224.8358 160.9605) (end 226.923 158.8733) (width 0.254) (layer B.Cu) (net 2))
 (segment (start 224.8358 180.8976) (end 224.8358 160.9605) (width 0.254) (layer B.Cu) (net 2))
 (segment (start 225.87 181.9318) (end 224.8358 180.8976) (width 0.254) (layer B.Cu) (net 2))
 (segment (start 225.87 183.62) (end 225.87 181.9318) (width 0.254) (layer B.Cu) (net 2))
 (segment (start 227.627 157.73) (end 227.627 158.8733) (width 0.254) (layer B.Cu) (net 2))
 (segment (start 226.0063 161.6367) (end 227.373 160.27) (width 0.254) (layer B.Cu) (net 3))
 (segment (start 226.0063 164.0485) (end 226.0063 161.6367) (width 0.254) (layer B.Cu) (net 3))
 (segment (start 227.3759 165.4181) (end 226.0063 164.0485) (width 0.254) (layer B.Cu) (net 3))
 (segment (start 227.3759 180.8977) (end 227.3759 165.4181) (width 0.254) (layer B.Cu) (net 3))
 (segment (start 228.41 181.9318) (end 227.3759 180.8977) (width 0.254) (layer B.Cu) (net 3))
 (segment (start 228.41 183.62) (end 228.41 181.9318) (width 0.254) (layer B.Cu) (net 3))
 (segment (start 280.6434 143.2936) (end 282.04 141.897) (width 0.254) (layer F.Cu) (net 14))
 (segment (start 280.6434 153.4076) (end 280.6434 143.2936) (width 0.254) (layer F.Cu) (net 14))
 (segment (start 270.32 163.731) (end 280.6434 153.4076) (width 0.254) (layer F.Cu) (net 14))
 (segment (start 270.32 171.7576) (end 270.32 163.731) (width 0.254) (layer F.Cu) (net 14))
 (segment (start 269.9388 172.1388) (end 270.32 171.7576) (width 0.254) (layer F.Cu) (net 14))
 (segment (start 272 174.2) (end 269.9388 172.1388) (width 0.254) (layer F.Cu) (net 14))
 (segment (start 246.19 183.62) (end 246.19 181.9318) (width 0.254) (layer F.Cu) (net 14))
 (segment (start 242.73 176) (end 244.087 176) (width 0.254) (layer F.Cu) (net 14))
 (segment (start 244.087 175.6426) (end 244.087 176) (width 0.254) (layer F.Cu) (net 14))
 (segment (start 247.5908 172.1388) (end 244.087 175.6426) (width 0.254) (layer F.Cu) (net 14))
 (segment (start 269.9388 172.1388) (end 247.5908 172.1388) (width 0.254) (layer F.Cu) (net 14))
 (segment (start 244.087 179.8288) (end 246.19 181.9318) (width 0.254) (layer F.Cu) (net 14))
 (segment (start 244.087 176) (end 244.087 179.8288) (width 0.254) (layer F.Cu) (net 14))
 (segment (start 243.65 183.62) (end 243.65 181.9318) (width 0.254) (layer F.Cu) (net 13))
 (segment (start 241.6184 179.9002) (end 243.65 181.9318) (width 0.254) (layer F.Cu) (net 13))
 (segment (start 241.6184 175.5844) (end 241.6184 179.9002) (width 0.254) (layer F.Cu) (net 13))
 (segment (start 246.1603 171.0425) (end 241.6184 175.5844) (width 0.254) (layer F.Cu) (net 13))
 (segment (start 248.2266 171.0425) (end 246.1603 171.0425) (width 0.254) (layer F.Cu) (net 13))
 (segment (start 250 169.2691) (end 248.2266 171.0425) (width 0.254) (layer F.Cu) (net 13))
 (segment (start 250 167.5004) (end 250 169.2691) (width 0.254) (layer F.Cu) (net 13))
 (segment (start 270.1624 147.338) (end 250 167.5004) (width 0.254) (layer F.Cu) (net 13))
 (segment (start 277.0467 147.338) (end 270.1624 147.338) (width 0.254) (layer F.Cu) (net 13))
 (segment (start 279.5 144.8847) (end 277.0467 147.338) (width 0.254) (layer F.Cu) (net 13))
 (segment (start 279.5 141.643) (end 279.5 144.8847) (width 0.254) (layer F.Cu) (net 13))
 (segment (start 271.59 165.5708) (end 271.59 168.38) (width 0.254) (layer B.Cu) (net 18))
 (segment (start 248.8545 142.8353) (end 271.59 165.5708) (width 0.254) (layer B.Cu) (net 18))
 (segment (start 246.041 142.8353) (end 248.8545 142.8353) (width 0.254) (layer B.Cu) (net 18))
 (segment (start 244.7933 141.5876) (end 246.041 142.8353) (width 0.254) (layer B.Cu) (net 18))
 (segment (start 244.7933 140.873) (end 244.7933 141.5876) (width 0.254) (layer B.Cu) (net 18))
 (segment (start 243.65 140.873) (end 244.7933 140.873) (width 0.254) (layer B.Cu) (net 18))
 (segment (start 266.6748 166.6918) (end 269.05 166.6918) (width 0.254) (layer B.Cu) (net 19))
 (segment (start 242.2533 142.2703) (end 266.6748 166.6918) (width 0.254) (layer B.Cu) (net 19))
 (segment (start 242.2533 141.127) (end 242.2533 142.2703) (width 0.254) (layer B.Cu) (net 19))
 (segment (start 241.11 141.127) (end 242.2533 141.127) (width 0.254) (layer B.Cu) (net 19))
 (segment (start 269.05 168.38) (end 269.05 166.6918) (width 0.254) (layer B.Cu) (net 19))
 (segment (start 256.5 181.7818) (end 256.5 178.54) (width 0.254) (layer B.Cu) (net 6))
 (segment (start 256.35 181.9318) (end 256.5 181.7818) (width 0.254) (layer B.Cu) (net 6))
 (segment (start 256.35 183.62) (end 256.35 181.9318) (width 0.254) (layer B.Cu) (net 6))
 (segment (start 253.81 176.15) (end 256.5 173.46) (width 0.254) (layer B.Cu) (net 5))
 (segment (start 253.81 183.62) (end 253.81 176.15) (width 0.254) (layer B.Cu) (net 5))
 (via (at 273.7917 179.5868) (size 0.889) (layers F.Cu B.Cu) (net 9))
 (segment (start 272.4634 180.9151) (end 273.7917 179.5868) (width 0.254) (layer F.Cu) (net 9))
 (segment (start 259.9067 180.9151) (end 272.4634 180.9151) (width 0.254) (layer F.Cu) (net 9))
 (segment (start 258.89 181.9318) (end 259.9067 180.9151) (width 0.254) (layer F.Cu) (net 9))
 (segment (start 275.9585 177.42) (end 279.627 177.42) (width 0.254) (layer B.Cu) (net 9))
 (segment (start 273.7917 179.5868) (end 275.9585 177.42) (width 0.254) (layer B.Cu) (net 9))
 (segment (start 258.89 183.62) (end 258.89 181.9318) (width 0.254) (layer F.Cu) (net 9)))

